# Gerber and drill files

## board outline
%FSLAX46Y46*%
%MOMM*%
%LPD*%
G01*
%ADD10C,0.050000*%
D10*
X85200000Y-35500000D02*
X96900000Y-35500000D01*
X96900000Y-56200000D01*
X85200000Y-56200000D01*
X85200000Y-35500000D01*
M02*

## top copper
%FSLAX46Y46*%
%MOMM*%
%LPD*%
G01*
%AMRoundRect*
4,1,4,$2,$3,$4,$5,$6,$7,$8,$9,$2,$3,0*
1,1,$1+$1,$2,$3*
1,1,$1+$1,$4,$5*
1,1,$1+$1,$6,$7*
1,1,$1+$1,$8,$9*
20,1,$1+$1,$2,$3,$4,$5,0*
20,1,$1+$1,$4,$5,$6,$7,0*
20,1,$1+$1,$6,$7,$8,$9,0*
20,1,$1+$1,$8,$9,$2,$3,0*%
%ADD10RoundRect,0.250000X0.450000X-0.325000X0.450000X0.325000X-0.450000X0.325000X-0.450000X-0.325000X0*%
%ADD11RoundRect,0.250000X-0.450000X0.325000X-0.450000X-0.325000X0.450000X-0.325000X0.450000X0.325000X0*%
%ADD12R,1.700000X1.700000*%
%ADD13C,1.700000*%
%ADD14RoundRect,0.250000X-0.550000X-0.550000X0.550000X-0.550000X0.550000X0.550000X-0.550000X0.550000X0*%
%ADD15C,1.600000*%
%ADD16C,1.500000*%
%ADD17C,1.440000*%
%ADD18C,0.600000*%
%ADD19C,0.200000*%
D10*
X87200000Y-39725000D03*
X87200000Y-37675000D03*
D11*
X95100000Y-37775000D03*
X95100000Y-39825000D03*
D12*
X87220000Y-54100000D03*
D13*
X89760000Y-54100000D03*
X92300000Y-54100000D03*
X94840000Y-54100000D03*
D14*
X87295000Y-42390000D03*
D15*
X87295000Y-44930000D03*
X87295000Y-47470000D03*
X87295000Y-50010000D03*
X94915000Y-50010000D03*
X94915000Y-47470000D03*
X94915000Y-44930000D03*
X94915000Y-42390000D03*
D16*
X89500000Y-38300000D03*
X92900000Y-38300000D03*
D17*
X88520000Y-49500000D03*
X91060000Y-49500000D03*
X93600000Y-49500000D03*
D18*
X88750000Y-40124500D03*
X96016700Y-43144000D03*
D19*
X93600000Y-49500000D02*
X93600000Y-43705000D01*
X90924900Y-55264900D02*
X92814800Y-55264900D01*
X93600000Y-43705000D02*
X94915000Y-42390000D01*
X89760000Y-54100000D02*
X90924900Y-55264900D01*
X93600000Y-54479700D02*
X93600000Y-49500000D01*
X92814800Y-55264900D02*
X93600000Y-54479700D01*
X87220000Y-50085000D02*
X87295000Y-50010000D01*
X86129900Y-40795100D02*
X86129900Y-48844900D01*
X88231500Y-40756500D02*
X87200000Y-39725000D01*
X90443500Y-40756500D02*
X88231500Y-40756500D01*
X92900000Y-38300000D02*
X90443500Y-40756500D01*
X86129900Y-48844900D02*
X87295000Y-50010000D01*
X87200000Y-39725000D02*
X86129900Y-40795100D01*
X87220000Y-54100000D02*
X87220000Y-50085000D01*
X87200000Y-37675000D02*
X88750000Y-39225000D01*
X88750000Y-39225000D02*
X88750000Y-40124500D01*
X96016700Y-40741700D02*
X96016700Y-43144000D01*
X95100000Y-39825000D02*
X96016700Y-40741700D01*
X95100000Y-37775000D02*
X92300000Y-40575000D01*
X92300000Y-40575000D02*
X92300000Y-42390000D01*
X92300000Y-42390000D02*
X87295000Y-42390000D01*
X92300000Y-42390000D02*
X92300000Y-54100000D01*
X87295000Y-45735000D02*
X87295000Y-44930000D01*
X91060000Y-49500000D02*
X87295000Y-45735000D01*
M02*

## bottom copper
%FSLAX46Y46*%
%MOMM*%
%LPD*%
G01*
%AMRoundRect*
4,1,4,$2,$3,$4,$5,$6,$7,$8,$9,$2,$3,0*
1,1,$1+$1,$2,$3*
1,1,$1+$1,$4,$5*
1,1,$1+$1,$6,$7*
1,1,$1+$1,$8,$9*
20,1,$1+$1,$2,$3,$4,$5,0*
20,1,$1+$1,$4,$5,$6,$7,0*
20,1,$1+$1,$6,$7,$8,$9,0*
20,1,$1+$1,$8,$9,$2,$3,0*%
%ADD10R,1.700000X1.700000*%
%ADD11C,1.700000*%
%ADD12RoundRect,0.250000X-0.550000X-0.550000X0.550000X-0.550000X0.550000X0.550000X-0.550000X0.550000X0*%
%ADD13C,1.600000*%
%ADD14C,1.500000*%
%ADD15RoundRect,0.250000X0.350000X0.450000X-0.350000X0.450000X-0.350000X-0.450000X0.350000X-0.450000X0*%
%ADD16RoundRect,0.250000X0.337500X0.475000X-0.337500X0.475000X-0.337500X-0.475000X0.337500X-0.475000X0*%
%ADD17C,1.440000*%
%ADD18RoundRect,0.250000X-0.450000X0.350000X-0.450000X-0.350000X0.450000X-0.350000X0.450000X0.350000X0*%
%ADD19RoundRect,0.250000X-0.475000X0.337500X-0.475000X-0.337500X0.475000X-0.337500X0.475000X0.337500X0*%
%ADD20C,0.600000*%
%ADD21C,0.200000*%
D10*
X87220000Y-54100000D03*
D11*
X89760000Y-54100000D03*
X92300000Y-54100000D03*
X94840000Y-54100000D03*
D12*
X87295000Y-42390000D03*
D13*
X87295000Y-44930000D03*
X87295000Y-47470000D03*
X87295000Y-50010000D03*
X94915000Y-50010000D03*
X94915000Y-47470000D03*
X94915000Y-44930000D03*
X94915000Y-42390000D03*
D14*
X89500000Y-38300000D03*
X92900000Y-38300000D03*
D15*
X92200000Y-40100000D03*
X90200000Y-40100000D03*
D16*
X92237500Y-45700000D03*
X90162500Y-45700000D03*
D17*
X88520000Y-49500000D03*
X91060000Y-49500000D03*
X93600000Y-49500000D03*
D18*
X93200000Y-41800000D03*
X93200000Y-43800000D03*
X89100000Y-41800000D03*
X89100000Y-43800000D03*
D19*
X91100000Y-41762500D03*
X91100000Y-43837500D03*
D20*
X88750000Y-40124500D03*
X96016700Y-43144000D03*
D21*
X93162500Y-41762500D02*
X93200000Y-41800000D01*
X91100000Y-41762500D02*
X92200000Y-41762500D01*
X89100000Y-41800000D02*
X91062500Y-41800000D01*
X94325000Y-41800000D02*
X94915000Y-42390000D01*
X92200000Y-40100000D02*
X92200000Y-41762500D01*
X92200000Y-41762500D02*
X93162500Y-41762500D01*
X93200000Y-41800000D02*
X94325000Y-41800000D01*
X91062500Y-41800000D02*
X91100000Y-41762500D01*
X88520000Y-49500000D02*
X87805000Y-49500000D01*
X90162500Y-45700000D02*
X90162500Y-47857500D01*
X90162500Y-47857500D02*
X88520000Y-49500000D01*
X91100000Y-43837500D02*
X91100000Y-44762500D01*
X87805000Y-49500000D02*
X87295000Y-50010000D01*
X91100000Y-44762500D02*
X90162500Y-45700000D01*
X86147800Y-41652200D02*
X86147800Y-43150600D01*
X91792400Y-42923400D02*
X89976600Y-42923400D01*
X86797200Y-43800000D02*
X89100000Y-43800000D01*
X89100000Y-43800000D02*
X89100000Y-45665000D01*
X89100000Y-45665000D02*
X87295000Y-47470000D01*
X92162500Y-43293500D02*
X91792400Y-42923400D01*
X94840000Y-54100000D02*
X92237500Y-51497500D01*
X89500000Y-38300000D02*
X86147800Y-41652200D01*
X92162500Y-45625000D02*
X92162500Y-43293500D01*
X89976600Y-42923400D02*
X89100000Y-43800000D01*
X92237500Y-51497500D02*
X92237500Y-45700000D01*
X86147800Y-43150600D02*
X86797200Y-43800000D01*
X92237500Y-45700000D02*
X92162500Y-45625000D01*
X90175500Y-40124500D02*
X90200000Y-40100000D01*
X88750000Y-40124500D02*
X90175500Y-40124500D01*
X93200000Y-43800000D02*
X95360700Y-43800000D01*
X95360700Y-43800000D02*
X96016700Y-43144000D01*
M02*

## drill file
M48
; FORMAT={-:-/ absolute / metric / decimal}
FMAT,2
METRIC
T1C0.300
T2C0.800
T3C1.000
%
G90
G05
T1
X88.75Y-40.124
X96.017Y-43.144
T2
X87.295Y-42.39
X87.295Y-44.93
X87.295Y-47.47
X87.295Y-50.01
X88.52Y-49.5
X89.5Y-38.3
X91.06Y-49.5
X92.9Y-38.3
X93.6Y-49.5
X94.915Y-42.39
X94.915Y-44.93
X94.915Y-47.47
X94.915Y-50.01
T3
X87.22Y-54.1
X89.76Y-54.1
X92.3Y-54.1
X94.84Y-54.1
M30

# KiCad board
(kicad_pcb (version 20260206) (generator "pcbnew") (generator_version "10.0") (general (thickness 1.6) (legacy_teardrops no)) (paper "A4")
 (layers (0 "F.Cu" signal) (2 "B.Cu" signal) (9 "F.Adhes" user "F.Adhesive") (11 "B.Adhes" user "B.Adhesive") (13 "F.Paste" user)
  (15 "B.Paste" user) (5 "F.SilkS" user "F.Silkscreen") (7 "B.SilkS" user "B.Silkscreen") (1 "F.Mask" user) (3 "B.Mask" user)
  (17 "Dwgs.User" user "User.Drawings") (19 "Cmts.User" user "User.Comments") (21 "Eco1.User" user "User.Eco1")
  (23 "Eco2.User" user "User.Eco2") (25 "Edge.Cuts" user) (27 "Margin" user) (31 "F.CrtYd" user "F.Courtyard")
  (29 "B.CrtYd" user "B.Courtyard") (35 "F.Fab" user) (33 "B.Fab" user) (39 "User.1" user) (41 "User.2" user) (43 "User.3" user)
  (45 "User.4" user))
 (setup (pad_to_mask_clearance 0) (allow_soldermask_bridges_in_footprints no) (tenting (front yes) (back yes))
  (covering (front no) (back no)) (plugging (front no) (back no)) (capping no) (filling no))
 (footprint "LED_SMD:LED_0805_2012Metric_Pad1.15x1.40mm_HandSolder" (layer "F.Cu") (at 87.2 38.7 90)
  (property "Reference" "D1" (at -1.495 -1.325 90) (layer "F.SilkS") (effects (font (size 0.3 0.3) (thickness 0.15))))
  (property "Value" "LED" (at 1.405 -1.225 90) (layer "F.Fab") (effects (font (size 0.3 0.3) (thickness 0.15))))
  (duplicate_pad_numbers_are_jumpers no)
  (pad "1" smd roundrect (at -1.025 0 90) (size 1.15 1.4) (layers "F.Cu" "F.Mask" "F.Paste") (roundrect_rratio 0.217391) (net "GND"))
  (pad "2" smd roundrect (at 1.025 0 90) (size 1.15 1.4) (layers "F.Cu" "F.Mask" "F.Paste") (roundrect_rratio 0.217391) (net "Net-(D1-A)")))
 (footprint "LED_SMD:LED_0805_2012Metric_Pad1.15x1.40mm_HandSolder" (layer "F.Cu") (at 95.1 38.8 -90)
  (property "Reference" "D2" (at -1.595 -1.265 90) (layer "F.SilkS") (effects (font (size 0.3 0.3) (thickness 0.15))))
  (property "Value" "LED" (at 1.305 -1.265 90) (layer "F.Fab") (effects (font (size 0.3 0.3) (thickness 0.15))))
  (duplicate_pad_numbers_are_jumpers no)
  (pad "1" smd roundrect (at -1.025 0 270) (size 1.15 1.4) (layers "F.Cu" "F.Mask" "F.Paste") (roundrect_rratio 0.217391) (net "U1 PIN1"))
  (pad "2" smd roundrect (at 1.025 0 270) (size 1.15 1.4) (layers "F.Cu" "F.Mask" "F.Paste") (roundrect_rratio 0.217391) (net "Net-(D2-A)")))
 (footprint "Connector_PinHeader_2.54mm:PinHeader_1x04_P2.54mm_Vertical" (layer "F.Cu") (at 87.22 54.1 90)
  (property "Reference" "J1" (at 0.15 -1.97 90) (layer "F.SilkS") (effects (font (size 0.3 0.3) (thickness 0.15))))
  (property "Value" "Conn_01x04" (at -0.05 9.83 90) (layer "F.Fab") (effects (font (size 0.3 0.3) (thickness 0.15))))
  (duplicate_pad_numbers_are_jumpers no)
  (pad "1" thru_hole rect (at 0 0 90) (size 1.7 1.7) (drill 1) (layers "*.Cu" "*.Mask") (remove_unused_layers no) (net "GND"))
  (pad "2" thru_hole circle (at 0 2.54 90) (size 1.7 1.7) (drill 1) (layers "*.Cu" "*.Mask") (remove_unused_layers no) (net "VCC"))
  (pad "3" thru_hole circle (at 0 5.08 90) (size 1.7 1.7) (drill 1) (layers "*.Cu" "*.Mask") (remove_unused_layers no) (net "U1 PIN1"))
  (pad "4" thru_hole circle (at 0 7.62 90) (size 1.7 1.7) (drill 1) (layers "*.Cu" "*.Mask") (remove_unused_layers no) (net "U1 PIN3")))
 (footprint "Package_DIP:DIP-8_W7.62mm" (layer "F.Cu") (at 87.295 42.39)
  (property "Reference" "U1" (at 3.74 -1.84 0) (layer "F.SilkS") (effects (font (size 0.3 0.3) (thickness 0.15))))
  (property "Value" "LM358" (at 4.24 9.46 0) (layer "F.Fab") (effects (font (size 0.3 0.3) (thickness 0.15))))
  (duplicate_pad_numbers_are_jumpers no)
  (pad "1" thru_hole roundrect (at 0 0) (size 1.6 1.6) (drill 0.8) (layers "*.Cu" "*.Mask") (remove_unused_layers no)
   (roundrect_rratio 0.15625) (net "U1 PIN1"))
  (pad "2" thru_hole circle (at 0 2.54) (size 1.6 1.6) (drill 0.8) (layers "*.Cu" "*.Mask") (remove_unused_layers no) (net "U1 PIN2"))
  (pad "3" thru_hole circle (at 0 5.08) (size 1.6 1.6) (drill 0.8) (layers "*.Cu" "*.Mask") (remove_unused_layers no) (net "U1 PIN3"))
  (pad "4" thru_hole circle (at 0 7.62) (size 1.6 1.6) (drill 0.8) (layers "*.Cu" "*.Mask") (remove_unused_layers no) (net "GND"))
  (pad "5" thru_hole circle (at 7.62 7.62) (size 1.6 1.6) (drill 0.8) (layers "*.Cu" "*.Mask") (remove_unused_layers no)
   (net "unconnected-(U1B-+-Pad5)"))
  (pad "6" thru_hole circle (at 7.62 5.08) (size 1.6 1.6) (drill 0.8) (layers "*.Cu" "*.Mask") (remove_unused_layers no)
   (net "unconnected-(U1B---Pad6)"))
  (pad "7" thru_hole circle (at 7.62 2.54) (size 1.6 1.6) (drill 0.8) (layers "*.Cu" "*.Mask") (remove_unused_layers no)
   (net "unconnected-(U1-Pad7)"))
  (pad "8" thru_hole circle (at 7.62 0) (size 1.6 1.6) (drill 0.8) (layers "*.Cu" "*.Mask") (remove_unused_layers no) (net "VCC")))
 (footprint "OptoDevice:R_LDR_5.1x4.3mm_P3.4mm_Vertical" (layer "F.Cu") (at 89.5 38.3)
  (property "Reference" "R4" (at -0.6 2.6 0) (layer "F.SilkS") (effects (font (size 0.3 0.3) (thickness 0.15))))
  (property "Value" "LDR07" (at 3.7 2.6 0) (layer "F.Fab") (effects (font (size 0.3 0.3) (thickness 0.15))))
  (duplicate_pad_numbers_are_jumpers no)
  (pad "1" thru_hole circle (at 0 0) (size 1.5 1.5) (drill 0.8) (layers "*.Cu" "*.Mask") (remove_unused_layers no) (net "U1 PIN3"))
  (pad "2" thru_hole circle (at 3.4 0) (size 1.5 1.5) (drill 0.8) (layers "*.Cu" "*.Mask") (remove_unused_layers no) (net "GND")))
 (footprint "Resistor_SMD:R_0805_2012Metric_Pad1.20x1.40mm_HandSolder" (layer "B.Cu") (at 91.2 40.1 180)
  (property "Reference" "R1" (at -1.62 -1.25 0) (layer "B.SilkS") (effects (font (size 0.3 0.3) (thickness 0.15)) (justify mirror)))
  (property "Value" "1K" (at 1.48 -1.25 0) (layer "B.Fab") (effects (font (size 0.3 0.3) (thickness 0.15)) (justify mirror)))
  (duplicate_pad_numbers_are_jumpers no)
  (pad "1" smd roundrect (at -1 0 180) (size 1.2 1.4) (layers "B.Cu" "B.Mask" "B.Paste") (roundrect_rratio 0.208333) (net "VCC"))
  (pad "2" smd roundrect (at 1 0 180) (size 1.2 1.4) (layers "B.Cu" "B.Mask" "B.Paste") (roundrect_rratio 0.208333) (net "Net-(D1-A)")))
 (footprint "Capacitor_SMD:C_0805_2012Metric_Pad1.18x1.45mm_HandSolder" (layer "B.Cu") (at 91.2 45.7 180)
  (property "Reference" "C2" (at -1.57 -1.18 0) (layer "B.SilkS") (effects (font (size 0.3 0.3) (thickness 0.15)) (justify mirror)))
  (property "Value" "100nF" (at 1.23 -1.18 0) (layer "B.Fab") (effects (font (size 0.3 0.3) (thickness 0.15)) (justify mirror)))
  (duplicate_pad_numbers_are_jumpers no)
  (pad "1" smd roundrect (at -1.0375 0 180) (size 1.175 1.45) (layers "B.Cu" "B.Mask" "B.Paste") (roundrect_rratio 0.212766) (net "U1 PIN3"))
  (pad "2" smd roundrect (at 1.0375 0 180) (size 1.175 1.45) (layers "B.Cu" "B.Mask" "B.Paste") (roundrect_rratio 0.212766) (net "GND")))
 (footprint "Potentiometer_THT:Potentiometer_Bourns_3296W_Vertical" (layer "B.Cu") (at 88.52 49.5 180)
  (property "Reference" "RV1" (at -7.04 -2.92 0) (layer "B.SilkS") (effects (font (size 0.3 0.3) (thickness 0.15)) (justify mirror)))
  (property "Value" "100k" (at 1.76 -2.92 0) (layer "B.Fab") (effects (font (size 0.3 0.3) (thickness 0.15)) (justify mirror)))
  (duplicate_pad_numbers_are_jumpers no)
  (pad "1" thru_hole circle (at 0 0 180) (size 1.44 1.44) (drill 0.8) (layers "*.Cu" "*.Mask") (remove_unused_layers no) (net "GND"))
  (pad "2" thru_hole circle (at -2.54 0 180) (size 1.44 1.44) (drill 0.8) (layers "*.Cu" "*.Mask") (remove_unused_layers no) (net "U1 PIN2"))
  (pad "3" thru_hole circle (at -5.08 0 180) (size 1.44 1.44) (drill 0.8) (layers "*.Cu" "*.Mask") (remove_unused_layers no) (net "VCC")))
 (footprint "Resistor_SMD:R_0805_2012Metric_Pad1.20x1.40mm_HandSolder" (layer "B.Cu") (at 93.2 42.8 -90)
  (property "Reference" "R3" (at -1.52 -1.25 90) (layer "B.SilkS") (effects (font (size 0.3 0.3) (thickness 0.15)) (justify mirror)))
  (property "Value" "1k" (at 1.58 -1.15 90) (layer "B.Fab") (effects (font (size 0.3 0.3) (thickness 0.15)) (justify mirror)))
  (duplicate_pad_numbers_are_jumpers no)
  (pad "1" smd roundrect (at -1 0 270) (size 1.2 1.4) (layers "B.Cu" "B.Mask" "B.Paste") (roundrect_rratio 0.208333) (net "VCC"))
  (pad "2" smd roundrect (at 1 0 270) (size 1.2 1.4) (layers "B.Cu" "B.Mask" "B.Paste") (roundrect_rratio 0.208333) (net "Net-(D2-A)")))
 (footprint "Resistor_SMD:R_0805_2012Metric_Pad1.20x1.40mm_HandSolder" (layer "B.Cu") (at 89.1 42.8 -90)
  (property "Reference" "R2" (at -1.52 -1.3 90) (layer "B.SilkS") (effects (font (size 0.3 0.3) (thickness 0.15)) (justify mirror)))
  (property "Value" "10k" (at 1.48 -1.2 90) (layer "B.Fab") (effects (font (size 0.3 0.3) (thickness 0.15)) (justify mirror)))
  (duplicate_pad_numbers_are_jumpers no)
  (pad "1" smd roundrect (at -1 0 270) (size 1.2 1.4) (layers "B.Cu" "B.Mask" "B.Paste") (roundrect_rratio 0.208333) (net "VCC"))
  (pad "2" smd roundrect (at 1 0 270) (size 1.2 1.4) (layers "B.Cu" "B.Mask" "B.Paste") (roundrect_rratio 0.208333) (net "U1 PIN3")))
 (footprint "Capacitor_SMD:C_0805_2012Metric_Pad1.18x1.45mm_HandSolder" (layer "B.Cu") (at 91.1 42.8 -90)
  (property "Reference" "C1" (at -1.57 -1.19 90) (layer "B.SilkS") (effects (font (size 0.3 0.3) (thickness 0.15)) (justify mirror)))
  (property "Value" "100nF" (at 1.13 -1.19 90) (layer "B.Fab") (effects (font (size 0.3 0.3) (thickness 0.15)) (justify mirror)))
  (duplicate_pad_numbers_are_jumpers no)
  (pad "1" smd roundrect (at -1.0375 0 270) (size 1.175 1.45) (layers "B.Cu" "B.Mask" "B.Paste") (roundrect_rratio 0.212766) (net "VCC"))
  (pad "2" smd roundrect (at 1.0375 0 270) (size 1.175 1.45) (layers "B.Cu" "B.Mask" "B.Paste") (roundrect_rratio 0.212766) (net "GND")))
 (gr_rect (start 85.2 35.5) (end 96.9 56.2) (stroke (width 0.05) (type default)) (fill no) (layer "Edge.Cuts"))
 (segment (start 93.6 49.5) (end 93.6 43.705) (width 0.2) (layer "F.Cu") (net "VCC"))
 (segment (start 90.9249 55.2649) (end 92.8148 55.2649) (width 0.2) (layer "F.Cu") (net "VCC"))
 (segment (start 93.6 43.705) (end 94.915 42.39) (width 0.2) (layer "F.Cu") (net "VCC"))
 (segment (start 89.76 54.1) (end 90.9249 55.2649) (width 0.2) (layer "F.Cu") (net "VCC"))
 (segment (start 93.6 54.4797) (end 93.6 49.5) (width 0.2) (layer "F.Cu") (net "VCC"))
 (segment (start 92.8148 55.2649) (end 93.6 54.4797) (width 0.2) (layer "F.Cu") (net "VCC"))
 (segment (start 93.1625 41.7625) (end 93.2 41.8) (width 0.2) (layer "B.Cu") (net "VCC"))
 (segment (start 91.1 41.7625) (end 92.2 41.7625) (width 0.2) (layer "B.Cu") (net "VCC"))
 (segment (start 89.1 41.8) (end 91.0625 41.8) (width 0.2) (layer "B.Cu") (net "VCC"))
 (segment (start 94.325 41.8) (end 94.915 42.39) (width 0.2) (layer "B.Cu") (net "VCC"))
 (segment (start 92.2 40.1) (end 92.2 41.7625) (width 0.2) (layer "B.Cu") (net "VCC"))
 (segment (start 92.2 41.7625) (end 93.1625 41.7625) (width 0.2) (layer "B.Cu") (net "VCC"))
 (segment (start 93.2 41.8) (end 94.325 41.8) (width 0.2) (layer "B.Cu") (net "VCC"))
 (segment (start 91.0625 41.8) (end 91.1 41.7625) (width 0.2) (layer "B.Cu") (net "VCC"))
 (segment (start 87.22 50.085) (end 87.295 50.01) (width 0.2) (layer "F.Cu") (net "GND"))
 (segment (start 86.1299 40.7951) (end 86.1299 48.8449) (width 0.2) (layer "F.Cu") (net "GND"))
 (segment (start 88.2315 40.7565) (end 87.2 39.725) (width 0.2) (layer "F.Cu") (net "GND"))
 (segment (start 90.4435 40.7565) (end 88.2315 40.7565) (width 0.2) (layer "F.Cu") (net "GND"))
 (segment (start 92.9 38.3) (end 90.4435 40.7565) (width 0.2) (layer "F.Cu") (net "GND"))
 (segment (start 86.1299 48.8449) (end 87.295 50.01) (width 0.2) (layer "F.Cu") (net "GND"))
 (segment (start 87.2 39.725) (end 86.1299 40.7951) (width 0.2) (layer "F.Cu") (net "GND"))
 (segment (start 87.22 54.1) (end 87.22 50.085) (width 0.2) (layer "F.Cu") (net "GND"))
 (segment (start 88.52 49.5) (end 87.805 49.5) (width 0.2) (layer "B.Cu") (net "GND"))
 (segment (start 90.1625 45.7) (end 90.1625 47.8575) (width 0.2) (layer "B.Cu") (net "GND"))
 (segment (start 90.1625 47.8575) (end 88.52 49.5) (width 0.2) (layer "B.Cu") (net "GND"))
 (segment (start 91.1 43.8375) (end 91.1 44.7625) (width 0.2) (layer "B.Cu") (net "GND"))
 (segment (start 87.805 49.5) (end 87.295 50.01) (width 0.2) (layer "B.Cu") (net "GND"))
 (segment (start 91.1 44.7625) (end 90.1625 45.7) (width 0.2) (layer "B.Cu") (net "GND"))
 (segment (start 86.1478 41.6522) (end 86.1478 43.1506) (width 0.2) (layer "B.Cu") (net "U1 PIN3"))
 (segment (start 91.7924 42.9234) (end 89.9766 42.9234) (width 0.2) (layer "B.Cu") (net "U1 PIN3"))
 (segment (start 86.7972 43.8) (end 89.1 43.8) (width 0.2) (layer "B.Cu") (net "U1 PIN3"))
 (segment (start 89.1 43.8) (end 89.1 45.665) (width 0.2) (layer "B.Cu") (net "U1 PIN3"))
 (segment (start 89.1 45.665) (end 87.295 47.47) (width 0.2) (layer "B.Cu") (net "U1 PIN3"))
 (segment (start 92.1625 43.2935) (end 91.7924 42.9234) (width 0.2) (layer "B.Cu") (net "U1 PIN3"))
 (segment (start 94.84 54.1) (end 92.2375 51.4975) (width 0.2) (layer "B.Cu") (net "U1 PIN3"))
 (segment (start 89.5 38.3) (end 86.1478 41.6522) (width 0.2) (layer "B.Cu") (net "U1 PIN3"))
 (segment (start 92.1625 45.625) (end 92.1625 43.2935) (width 0.2) (layer "B.Cu") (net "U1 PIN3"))
 (segment (start 89.9766 42.9234) (end 89.1 43.8) (width 0.2) (layer "B.Cu") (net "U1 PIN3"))
 (segment (start 92.2375 51.4975) (end 92.2375 45.7) (width 0.2) (layer "B.Cu") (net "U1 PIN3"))
 (segment (start 86.1478 43.1506) (end 86.7972 43.8) (width 0.2) (layer "B.Cu") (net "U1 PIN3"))
 (segment (start 92.2375 45.7) (end 92.1625 45.625) (width 0.2) (layer "B.Cu") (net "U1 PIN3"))
 (segment (start 87.2 37.675) (end 88.75 39.225) (width 0.2) (layer "F.Cu") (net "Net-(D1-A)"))
 (segment (start 88.75 39.225) (end 88.75 40.1245) (width 0.2) (layer "F.Cu") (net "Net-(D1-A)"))
 (via (at 88.75 40.1245) (size 0.6) (drill 0.3) (layers "F.Cu" "B.Cu") (capping no) (covering (front no) (back no))
  (plugging (front no) (back no)) (filling no) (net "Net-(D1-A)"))
 (segment (start 90.1755 40.1245) (end 90.2 40.1) (width 0.2) (layer "B.Cu") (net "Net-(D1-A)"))
 (segment (start 88.75 40.1245) (end 90.1755 40.1245) (width 0.2) (layer "B.Cu") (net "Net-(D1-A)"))
 (segment (start 96.0167 40.7417) (end 96.0167 43.144) (width 0.2) (layer "F.Cu") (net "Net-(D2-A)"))
 (segment (start 95.1 39.825) (end 96.0167 40.7417) (width 0.2) (layer "F.Cu") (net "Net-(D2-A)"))
 (via (at 96.0167 43.144) (size 0.6) (drill 0.3) (layers "F.Cu" "B.Cu") (capping no) (covering (front no) (back no))
  (plugging (front no) (back no)) (filling no) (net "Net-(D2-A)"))
 (segment (start 93.2 43.8) (end 95.3607 43.8) (width 0.2) (layer "B.Cu") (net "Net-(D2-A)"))
 (segment (start 95.3607 43.8) (end 96.0167 43.144) (width 0.2) (layer "B.Cu") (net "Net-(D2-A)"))
 (segment (start 95.1 37.775) (end 92.3 40.575) (width 0.2) (layer "F.Cu") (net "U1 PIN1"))
 (segment (start 92.3 40.575) (end 92.3 42.39) (width 0.2) (layer "F.Cu") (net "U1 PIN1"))
 (segment (start 92.3 42.39) (end 87.295 42.39) (width 0.2) (layer "F.Cu") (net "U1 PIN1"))
 (segment (start 92.3 42.39) (end 92.3 54.1) (width 0.2) (layer "F.Cu") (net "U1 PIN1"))
 (segment (start 87.295 45.735) (end 87.295 44.93) (width 0.2) (layer "F.Cu") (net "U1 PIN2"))
 (segment (start 91.06 49.5) (end 87.295 45.735) (width 0.2) (layer "F.Cu") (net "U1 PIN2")))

